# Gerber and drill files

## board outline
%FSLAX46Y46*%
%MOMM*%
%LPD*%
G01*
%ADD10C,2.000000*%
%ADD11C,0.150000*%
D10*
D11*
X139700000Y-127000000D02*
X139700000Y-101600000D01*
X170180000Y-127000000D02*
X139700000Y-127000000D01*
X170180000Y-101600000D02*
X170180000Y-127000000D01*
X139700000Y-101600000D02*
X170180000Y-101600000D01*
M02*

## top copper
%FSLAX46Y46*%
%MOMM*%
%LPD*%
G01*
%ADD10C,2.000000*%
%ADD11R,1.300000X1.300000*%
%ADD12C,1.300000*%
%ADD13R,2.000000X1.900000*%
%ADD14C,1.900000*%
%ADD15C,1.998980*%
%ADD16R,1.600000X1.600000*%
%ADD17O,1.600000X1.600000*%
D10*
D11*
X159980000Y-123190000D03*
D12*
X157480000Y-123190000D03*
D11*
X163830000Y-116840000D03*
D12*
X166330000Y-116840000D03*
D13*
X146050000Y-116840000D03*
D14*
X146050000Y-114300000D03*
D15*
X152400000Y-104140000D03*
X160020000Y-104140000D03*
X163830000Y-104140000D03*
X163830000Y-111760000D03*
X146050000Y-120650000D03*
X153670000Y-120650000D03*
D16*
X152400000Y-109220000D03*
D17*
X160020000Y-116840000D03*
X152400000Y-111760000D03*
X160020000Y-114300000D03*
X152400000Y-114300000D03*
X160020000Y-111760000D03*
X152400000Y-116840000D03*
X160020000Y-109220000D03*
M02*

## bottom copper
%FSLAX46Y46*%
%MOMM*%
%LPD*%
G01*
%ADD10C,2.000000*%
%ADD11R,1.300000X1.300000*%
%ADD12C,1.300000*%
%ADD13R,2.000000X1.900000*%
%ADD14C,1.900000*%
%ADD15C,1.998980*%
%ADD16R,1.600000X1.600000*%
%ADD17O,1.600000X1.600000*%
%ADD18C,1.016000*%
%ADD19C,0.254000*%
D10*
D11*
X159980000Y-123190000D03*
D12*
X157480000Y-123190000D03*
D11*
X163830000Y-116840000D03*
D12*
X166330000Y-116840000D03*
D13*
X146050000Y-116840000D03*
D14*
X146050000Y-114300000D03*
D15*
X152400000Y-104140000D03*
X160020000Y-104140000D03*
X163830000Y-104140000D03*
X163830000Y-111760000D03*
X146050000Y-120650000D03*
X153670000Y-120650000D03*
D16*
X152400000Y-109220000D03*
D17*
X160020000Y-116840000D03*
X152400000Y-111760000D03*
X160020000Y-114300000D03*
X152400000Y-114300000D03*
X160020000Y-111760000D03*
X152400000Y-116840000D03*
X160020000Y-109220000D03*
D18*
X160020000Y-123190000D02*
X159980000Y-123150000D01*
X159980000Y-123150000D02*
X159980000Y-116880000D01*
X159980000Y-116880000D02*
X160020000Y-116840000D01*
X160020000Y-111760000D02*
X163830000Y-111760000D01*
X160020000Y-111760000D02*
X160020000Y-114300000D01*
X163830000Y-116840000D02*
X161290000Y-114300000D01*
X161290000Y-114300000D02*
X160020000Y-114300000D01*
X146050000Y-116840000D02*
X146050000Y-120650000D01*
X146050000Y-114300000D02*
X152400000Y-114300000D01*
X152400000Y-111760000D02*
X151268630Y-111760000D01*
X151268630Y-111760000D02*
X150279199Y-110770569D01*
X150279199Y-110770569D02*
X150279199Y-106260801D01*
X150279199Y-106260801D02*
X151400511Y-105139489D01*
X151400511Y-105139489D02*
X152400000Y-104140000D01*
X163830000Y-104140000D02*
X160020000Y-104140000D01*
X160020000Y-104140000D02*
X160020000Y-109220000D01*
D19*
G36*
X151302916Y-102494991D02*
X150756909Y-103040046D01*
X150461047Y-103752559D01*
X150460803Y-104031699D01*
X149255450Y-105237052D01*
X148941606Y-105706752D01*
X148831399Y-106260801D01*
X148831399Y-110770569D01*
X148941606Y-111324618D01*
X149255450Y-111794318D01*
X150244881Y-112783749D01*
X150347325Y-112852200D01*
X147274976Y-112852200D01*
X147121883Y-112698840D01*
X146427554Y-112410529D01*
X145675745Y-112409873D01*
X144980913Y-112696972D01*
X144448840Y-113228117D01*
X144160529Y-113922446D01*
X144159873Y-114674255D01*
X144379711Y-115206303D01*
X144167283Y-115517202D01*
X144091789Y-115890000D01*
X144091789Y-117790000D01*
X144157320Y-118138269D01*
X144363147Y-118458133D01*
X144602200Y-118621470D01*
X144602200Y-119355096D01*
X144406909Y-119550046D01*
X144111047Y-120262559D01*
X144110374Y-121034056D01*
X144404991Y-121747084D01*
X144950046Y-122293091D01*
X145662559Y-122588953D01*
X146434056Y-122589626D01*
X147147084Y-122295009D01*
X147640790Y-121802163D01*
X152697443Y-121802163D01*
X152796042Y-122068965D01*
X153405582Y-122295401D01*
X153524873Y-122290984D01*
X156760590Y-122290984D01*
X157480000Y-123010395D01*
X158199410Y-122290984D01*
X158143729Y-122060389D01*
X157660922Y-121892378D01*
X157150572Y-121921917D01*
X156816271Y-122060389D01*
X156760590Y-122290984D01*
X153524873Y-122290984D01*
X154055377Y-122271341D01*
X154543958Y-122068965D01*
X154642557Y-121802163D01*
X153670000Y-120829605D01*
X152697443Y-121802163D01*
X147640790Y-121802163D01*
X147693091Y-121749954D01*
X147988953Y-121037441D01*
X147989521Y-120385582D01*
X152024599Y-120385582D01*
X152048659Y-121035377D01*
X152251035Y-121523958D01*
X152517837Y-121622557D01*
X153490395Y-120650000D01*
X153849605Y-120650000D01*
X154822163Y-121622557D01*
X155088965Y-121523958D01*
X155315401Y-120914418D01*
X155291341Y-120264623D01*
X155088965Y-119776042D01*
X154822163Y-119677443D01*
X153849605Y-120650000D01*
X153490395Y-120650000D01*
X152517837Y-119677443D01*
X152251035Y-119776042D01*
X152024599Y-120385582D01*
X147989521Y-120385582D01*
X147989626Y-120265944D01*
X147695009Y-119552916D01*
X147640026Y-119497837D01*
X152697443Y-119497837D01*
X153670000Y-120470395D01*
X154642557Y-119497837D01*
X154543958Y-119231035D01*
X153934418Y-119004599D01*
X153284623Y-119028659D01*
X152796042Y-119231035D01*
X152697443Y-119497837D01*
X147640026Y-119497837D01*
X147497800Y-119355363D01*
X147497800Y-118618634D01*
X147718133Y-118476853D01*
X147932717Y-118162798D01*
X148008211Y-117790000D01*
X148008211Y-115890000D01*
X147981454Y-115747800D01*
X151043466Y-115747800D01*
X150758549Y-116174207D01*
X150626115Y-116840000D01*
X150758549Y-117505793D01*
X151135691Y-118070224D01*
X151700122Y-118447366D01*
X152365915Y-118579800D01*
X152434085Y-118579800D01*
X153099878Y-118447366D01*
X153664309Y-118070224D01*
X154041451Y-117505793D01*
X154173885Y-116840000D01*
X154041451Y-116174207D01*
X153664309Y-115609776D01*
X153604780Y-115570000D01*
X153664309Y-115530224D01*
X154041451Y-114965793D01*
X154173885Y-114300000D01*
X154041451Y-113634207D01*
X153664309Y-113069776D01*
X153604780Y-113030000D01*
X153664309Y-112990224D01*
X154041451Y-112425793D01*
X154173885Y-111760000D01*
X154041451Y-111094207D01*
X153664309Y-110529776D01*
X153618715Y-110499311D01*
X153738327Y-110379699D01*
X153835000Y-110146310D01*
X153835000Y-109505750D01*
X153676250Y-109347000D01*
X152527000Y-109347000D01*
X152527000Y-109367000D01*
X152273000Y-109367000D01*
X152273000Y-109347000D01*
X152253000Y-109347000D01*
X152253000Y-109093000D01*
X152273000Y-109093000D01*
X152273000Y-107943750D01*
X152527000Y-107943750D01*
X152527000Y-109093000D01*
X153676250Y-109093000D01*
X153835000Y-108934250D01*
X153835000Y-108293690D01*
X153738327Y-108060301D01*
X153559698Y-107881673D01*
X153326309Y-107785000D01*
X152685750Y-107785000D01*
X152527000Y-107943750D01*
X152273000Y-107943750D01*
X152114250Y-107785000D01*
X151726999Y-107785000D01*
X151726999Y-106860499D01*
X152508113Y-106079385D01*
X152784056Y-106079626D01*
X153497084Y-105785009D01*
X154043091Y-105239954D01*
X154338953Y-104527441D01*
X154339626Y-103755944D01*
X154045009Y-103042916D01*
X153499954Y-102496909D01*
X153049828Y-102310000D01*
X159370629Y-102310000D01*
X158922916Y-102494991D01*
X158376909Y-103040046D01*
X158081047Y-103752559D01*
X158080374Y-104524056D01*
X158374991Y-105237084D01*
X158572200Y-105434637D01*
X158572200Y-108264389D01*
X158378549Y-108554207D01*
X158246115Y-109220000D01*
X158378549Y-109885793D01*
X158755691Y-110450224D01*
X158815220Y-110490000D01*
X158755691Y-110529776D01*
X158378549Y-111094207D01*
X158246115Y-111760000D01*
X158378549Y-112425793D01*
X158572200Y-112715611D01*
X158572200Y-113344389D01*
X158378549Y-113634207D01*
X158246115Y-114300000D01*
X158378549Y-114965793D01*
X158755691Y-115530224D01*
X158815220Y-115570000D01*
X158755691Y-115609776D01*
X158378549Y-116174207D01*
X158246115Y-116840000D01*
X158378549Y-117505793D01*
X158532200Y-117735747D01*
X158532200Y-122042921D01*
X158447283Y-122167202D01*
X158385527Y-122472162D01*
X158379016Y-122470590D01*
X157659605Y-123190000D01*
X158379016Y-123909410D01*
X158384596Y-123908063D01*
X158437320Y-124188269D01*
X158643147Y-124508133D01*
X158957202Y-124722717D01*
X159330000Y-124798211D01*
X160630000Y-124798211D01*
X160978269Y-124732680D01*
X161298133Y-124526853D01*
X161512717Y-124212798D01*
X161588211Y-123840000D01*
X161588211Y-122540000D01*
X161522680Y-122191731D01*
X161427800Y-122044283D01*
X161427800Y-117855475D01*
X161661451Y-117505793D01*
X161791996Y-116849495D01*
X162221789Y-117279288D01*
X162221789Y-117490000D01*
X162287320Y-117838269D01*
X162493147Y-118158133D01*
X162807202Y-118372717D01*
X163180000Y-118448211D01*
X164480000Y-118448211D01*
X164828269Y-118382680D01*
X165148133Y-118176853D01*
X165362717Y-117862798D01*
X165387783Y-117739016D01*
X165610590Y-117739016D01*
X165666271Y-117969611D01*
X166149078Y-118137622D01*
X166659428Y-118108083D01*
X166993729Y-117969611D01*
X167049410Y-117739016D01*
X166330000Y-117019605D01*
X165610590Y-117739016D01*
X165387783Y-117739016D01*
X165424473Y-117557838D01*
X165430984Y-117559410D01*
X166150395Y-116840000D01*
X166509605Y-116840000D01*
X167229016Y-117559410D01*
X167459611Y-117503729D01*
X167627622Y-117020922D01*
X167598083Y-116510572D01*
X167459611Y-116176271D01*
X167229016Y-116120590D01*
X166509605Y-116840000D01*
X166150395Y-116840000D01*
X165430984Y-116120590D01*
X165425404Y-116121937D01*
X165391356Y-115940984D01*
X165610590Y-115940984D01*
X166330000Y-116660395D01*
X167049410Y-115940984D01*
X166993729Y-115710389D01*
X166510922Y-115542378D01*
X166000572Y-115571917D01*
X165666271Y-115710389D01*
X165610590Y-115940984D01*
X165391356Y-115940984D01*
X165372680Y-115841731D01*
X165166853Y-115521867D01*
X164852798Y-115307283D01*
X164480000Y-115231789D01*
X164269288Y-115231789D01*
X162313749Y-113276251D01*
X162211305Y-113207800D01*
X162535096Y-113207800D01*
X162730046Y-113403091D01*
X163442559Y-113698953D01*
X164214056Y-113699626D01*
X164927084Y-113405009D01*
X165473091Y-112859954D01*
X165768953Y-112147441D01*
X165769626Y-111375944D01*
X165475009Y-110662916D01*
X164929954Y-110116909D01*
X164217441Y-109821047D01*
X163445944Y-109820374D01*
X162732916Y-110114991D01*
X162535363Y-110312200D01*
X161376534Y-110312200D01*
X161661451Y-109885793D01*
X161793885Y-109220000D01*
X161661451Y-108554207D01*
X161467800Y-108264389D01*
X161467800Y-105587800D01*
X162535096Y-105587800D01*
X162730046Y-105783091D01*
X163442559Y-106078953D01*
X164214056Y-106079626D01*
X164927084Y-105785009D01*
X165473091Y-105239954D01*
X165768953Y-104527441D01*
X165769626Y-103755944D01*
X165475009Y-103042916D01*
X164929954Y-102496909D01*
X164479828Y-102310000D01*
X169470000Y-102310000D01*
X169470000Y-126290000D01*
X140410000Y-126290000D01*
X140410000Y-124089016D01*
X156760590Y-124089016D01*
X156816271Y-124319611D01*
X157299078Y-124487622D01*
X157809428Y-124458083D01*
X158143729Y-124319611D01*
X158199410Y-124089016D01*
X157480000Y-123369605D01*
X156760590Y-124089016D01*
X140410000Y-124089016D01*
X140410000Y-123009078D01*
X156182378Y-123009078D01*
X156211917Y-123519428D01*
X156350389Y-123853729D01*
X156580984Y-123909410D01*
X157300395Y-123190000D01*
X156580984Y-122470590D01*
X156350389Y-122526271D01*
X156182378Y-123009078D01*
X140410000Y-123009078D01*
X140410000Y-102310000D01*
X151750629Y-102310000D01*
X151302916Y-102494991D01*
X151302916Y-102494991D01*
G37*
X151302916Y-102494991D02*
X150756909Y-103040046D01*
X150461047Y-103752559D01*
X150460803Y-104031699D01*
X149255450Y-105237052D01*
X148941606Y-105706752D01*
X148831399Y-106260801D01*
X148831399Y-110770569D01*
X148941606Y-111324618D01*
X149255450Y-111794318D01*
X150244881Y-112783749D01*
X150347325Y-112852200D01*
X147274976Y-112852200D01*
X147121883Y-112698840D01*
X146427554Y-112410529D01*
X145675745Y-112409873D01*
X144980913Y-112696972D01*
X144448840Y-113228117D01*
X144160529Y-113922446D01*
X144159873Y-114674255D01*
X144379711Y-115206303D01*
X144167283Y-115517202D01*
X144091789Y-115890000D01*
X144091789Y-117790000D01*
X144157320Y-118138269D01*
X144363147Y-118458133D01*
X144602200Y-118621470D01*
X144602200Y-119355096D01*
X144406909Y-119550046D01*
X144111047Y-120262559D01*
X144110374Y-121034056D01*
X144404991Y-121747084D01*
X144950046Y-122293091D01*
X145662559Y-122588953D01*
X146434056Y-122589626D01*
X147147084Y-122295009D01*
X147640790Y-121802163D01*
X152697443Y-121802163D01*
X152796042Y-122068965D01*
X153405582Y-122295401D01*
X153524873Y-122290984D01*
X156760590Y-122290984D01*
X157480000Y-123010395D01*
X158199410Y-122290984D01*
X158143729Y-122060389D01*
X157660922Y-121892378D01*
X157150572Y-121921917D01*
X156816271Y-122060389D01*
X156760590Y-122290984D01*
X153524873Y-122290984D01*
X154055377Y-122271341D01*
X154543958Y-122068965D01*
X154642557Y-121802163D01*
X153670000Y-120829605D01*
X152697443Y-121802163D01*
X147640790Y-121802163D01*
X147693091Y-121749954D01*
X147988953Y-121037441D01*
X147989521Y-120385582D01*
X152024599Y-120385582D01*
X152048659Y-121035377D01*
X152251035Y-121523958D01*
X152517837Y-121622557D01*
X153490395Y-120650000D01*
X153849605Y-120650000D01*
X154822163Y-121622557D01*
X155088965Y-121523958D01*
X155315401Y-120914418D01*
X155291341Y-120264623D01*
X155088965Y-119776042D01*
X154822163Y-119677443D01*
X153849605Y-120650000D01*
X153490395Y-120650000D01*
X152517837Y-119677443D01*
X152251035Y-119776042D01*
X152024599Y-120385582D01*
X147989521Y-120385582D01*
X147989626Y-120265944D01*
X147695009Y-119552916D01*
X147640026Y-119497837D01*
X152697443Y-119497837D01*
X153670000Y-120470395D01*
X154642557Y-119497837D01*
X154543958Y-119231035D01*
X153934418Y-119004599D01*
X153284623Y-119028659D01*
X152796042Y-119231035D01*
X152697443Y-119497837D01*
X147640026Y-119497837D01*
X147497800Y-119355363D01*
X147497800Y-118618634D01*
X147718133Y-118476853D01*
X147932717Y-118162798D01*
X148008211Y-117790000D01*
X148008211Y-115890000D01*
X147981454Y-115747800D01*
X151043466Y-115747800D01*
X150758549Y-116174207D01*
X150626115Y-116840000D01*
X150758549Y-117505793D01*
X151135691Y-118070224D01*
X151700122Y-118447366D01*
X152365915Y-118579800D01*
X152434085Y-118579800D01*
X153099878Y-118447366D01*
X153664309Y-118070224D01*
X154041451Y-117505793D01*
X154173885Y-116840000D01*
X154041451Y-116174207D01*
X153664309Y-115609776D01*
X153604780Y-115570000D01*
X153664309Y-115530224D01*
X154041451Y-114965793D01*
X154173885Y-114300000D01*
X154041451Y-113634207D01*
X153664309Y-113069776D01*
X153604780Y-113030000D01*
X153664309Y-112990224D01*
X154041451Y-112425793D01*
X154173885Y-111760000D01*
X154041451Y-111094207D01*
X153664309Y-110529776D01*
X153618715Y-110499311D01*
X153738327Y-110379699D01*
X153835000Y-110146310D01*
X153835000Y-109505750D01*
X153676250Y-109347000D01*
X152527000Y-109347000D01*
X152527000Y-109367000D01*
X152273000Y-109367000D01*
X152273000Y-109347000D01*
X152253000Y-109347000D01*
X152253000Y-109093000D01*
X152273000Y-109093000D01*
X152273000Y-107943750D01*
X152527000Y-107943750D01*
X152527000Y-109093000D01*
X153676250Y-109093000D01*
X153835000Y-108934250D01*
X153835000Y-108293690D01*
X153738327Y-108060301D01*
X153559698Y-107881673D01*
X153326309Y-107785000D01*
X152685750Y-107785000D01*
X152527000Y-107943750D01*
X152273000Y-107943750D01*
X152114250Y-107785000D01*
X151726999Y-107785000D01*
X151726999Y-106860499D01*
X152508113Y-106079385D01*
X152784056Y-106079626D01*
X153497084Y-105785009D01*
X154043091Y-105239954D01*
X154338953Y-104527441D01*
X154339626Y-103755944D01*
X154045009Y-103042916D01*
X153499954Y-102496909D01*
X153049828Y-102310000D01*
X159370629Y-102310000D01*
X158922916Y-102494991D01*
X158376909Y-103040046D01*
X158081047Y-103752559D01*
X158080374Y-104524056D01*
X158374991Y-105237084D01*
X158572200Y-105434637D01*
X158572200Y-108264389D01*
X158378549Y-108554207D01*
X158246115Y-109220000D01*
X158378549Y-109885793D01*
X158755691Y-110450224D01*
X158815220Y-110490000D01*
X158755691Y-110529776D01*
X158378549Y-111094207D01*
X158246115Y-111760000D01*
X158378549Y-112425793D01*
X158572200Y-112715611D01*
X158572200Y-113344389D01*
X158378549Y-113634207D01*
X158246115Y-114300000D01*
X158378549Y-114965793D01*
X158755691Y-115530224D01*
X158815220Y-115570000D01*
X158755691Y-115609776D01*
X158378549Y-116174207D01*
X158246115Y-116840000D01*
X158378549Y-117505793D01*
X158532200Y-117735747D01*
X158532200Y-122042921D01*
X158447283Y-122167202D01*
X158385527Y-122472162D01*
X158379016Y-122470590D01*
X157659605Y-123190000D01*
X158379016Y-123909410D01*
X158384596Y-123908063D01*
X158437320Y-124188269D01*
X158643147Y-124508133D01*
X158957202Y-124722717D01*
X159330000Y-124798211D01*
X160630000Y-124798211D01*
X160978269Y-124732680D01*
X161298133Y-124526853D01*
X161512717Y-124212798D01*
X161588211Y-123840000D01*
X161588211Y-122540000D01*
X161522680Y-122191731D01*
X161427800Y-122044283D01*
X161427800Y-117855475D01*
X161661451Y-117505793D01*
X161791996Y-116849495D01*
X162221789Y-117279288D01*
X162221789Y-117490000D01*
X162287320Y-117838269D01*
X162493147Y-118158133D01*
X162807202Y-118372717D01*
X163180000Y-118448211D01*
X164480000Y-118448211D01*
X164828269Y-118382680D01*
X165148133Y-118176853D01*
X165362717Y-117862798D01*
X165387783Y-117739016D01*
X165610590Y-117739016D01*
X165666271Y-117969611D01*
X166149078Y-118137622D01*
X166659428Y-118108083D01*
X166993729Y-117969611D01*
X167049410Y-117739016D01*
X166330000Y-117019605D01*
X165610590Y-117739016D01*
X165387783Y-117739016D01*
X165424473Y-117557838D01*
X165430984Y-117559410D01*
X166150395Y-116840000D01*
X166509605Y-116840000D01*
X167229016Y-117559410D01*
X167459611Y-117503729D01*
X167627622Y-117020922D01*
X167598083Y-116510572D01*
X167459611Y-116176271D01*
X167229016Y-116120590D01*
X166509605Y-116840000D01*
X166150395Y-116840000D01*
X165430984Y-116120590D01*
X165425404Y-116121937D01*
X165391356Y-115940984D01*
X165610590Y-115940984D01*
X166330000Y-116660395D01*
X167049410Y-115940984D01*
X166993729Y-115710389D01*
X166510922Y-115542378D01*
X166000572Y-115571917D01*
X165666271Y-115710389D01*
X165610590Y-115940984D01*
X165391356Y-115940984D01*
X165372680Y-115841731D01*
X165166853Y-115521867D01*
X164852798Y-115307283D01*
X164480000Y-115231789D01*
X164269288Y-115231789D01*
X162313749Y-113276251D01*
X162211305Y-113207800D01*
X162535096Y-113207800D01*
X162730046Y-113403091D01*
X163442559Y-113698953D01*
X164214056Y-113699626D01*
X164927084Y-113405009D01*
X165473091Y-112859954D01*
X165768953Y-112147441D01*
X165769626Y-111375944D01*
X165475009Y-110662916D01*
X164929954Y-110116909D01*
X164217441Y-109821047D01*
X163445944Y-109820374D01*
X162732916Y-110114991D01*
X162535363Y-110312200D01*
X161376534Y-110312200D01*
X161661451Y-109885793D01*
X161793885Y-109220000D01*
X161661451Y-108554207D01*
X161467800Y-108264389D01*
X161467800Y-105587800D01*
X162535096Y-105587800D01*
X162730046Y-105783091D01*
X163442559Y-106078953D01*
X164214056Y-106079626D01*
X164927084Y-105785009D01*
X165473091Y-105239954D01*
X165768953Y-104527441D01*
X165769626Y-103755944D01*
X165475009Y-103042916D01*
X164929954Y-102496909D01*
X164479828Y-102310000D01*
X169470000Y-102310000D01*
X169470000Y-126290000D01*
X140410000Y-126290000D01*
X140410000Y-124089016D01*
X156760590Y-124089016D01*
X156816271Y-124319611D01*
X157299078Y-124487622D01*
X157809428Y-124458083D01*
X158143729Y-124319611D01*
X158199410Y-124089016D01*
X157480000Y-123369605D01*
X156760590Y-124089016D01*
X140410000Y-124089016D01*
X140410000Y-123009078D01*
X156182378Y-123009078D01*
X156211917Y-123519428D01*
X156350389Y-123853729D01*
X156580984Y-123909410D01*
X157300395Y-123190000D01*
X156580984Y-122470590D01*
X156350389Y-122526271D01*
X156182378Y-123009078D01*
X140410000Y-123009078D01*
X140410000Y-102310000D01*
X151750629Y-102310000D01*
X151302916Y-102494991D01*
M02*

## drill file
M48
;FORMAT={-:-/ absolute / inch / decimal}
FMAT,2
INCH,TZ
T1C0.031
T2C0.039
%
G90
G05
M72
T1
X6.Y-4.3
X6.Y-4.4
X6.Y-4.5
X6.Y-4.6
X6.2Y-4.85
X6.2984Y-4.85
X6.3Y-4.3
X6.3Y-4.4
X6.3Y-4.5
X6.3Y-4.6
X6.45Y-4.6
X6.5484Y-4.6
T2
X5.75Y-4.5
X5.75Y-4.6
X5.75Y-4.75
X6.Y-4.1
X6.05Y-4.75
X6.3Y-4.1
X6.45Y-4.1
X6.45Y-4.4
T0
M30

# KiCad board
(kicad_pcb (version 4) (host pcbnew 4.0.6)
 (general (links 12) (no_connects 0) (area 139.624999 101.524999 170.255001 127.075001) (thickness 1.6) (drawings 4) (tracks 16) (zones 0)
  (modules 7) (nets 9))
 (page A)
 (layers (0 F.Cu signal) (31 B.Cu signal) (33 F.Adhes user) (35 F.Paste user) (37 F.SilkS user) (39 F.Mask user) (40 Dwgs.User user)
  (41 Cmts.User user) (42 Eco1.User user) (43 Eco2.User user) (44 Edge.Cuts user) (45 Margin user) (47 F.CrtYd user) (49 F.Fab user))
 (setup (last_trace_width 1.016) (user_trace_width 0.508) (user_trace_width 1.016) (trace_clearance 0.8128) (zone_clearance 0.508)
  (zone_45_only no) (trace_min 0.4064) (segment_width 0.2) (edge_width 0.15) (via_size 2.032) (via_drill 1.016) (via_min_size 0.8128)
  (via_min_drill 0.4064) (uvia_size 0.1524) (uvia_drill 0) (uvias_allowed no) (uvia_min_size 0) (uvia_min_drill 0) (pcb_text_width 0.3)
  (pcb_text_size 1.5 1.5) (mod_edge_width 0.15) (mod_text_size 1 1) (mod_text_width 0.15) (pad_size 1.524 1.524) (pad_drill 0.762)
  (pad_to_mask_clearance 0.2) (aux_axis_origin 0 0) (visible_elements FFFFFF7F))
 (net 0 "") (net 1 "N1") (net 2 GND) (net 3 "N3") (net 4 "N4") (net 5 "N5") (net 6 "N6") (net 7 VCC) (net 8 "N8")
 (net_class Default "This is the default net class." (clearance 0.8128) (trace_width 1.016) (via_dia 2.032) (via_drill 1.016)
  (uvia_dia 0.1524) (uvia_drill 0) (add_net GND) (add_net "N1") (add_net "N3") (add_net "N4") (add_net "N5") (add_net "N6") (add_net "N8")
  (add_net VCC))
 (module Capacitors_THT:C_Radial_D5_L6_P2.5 (layer F.Cu) (at 159.98 123.19 180)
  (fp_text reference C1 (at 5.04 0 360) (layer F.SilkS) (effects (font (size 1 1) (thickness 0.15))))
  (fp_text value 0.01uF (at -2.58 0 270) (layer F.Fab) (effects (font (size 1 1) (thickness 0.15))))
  (pad 1 thru_hole rect (at 0 0 180) (size 1.3 1.3) (drill 0.8) (layers *.Cu *.Mask) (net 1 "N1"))
  (pad 2 thru_hole circle (at 2.5 0 180) (size 1.3 1.3) (drill 0.8) (layers *.Cu *.Mask) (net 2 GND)))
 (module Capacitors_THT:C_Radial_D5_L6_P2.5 (layer F.Cu) (at 163.83 116.84)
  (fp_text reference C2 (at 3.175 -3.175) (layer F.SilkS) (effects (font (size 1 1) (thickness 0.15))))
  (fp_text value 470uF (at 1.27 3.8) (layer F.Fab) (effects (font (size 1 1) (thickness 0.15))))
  (pad 1 thru_hole rect (at 0 0) (size 1.3 1.3) (drill 0.8) (layers *.Cu *.Mask) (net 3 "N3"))
  (pad 2 thru_hole circle (at 2.5 0) (size 1.3 1.3) (drill 0.8) (layers *.Cu *.Mask) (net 2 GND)))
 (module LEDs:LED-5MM (layer F.Cu) (at 146.05 116.84 90)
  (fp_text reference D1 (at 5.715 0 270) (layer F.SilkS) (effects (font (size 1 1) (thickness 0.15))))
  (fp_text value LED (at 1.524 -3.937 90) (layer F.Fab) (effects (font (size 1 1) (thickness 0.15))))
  (pad 1 thru_hole rect (at 0 0 180) (size 2 1.9) (drill 1.00076) (layers *.Cu *.Mask) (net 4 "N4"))
  (pad 2 thru_hole circle (at 2.54 0 90) (size 1.9 1.9) (drill 1.00076) (layers *.Cu *.Mask) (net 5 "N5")))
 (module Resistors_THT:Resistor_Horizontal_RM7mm (layer F.Cu) (at 152.4 104.14)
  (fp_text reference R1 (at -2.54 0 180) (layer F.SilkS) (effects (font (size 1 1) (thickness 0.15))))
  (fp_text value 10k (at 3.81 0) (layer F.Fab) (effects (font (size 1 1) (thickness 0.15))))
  (pad 1 thru_hole circle (at 0 0) (size 1.99898 1.99898) (drill 1.00076) (layers *.Cu *.SilkS *.Mask) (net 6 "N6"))
  (pad 2 thru_hole circle (at 7.62 0) (size 1.99898 1.99898) (drill 1.00076) (layers *.Cu *.SilkS *.Mask) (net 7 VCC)))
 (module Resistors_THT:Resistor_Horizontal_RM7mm (layer F.Cu) (at 163.83 104.14 270)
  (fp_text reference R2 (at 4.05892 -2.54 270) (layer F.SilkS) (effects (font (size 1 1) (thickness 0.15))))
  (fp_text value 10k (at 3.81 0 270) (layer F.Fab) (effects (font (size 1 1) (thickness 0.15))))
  (pad 1 thru_hole circle (at 0 0 270) (size 1.99898 1.99898) (drill 1.00076) (layers *.Cu *.SilkS *.Mask) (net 7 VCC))
  (pad 2 thru_hole circle (at 7.62 0 270) (size 1.99898 1.99898) (drill 1.00076) (layers *.Cu *.SilkS *.Mask) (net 3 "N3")))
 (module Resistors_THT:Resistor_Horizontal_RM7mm (layer F.Cu) (at 146.05 120.65)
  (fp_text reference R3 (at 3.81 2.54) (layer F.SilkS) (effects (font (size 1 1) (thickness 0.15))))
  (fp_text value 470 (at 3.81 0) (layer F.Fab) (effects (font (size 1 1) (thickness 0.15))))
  (pad 1 thru_hole circle (at 0 0) (size 1.99898 1.99898) (drill 1.00076) (layers *.Cu *.SilkS *.Mask) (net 4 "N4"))
  (pad 2 thru_hole circle (at 7.62 0) (size 1.99898 1.99898) (drill 1.00076) (layers *.Cu *.SilkS *.Mask) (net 2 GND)))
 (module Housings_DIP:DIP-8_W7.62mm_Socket (layer F.Cu) (at 152.4 109.22)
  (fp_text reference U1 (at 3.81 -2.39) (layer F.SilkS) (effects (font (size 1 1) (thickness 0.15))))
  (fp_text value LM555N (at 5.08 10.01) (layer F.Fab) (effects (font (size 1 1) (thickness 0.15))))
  (pad 1 thru_hole rect (at 0 0) (size 1.6 1.6) (drill 0.8) (layers *.Cu *.Mask) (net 2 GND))
  (pad 5 thru_hole oval (at 7.62 7.62) (size 1.6 1.6) (drill 0.8) (layers *.Cu *.Mask) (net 1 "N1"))
  (pad 2 thru_hole oval (at 0 2.54) (size 1.6 1.6) (drill 0.8) (layers *.Cu *.Mask) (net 6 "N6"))
  (pad 6 thru_hole oval (at 7.62 5.08) (size 1.6 1.6) (drill 0.8) (layers *.Cu *.Mask) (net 3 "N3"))
  (pad 3 thru_hole oval (at 0 5.08) (size 1.6 1.6) (drill 0.8) (layers *.Cu *.Mask) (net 5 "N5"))
  (pad 7 thru_hole oval (at 7.62 2.54) (size 1.6 1.6) (drill 0.8) (layers *.Cu *.Mask) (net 3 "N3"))
  (pad 4 thru_hole oval (at 0 7.62) (size 1.6 1.6) (drill 0.8) (layers *.Cu *.Mask) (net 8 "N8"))
  (pad 8 thru_hole oval (at 7.62 0) (size 1.6 1.6) (drill 0.8) (layers *.Cu *.Mask) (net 7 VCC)))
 (gr_line (start 139.7 127) (end 139.7 101.6) (layer Edge.Cuts) (width 0.15))
 (gr_line (start 170.18 127) (end 139.7 127) (layer Edge.Cuts) (width 0.15))
 (gr_line (start 170.18 101.6) (end 170.18 127) (layer Edge.Cuts) (width 0.15))
 (gr_line (start 139.7 101.6) (end 170.18 101.6) (layer Edge.Cuts) (width 0.15))
 (segment (start 160.02 123.19) (end 159.98 123.15) (width 1.016) (layer B.Cu) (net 1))
 (segment (start 159.98 123.15) (end 159.98 116.88) (width 1.016) (layer B.Cu) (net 1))
 (segment (start 159.98 116.88) (end 160.02 116.84) (width 1.016) (layer B.Cu) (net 1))
 (segment (start 160.02 111.76) (end 163.83 111.76) (width 1.016) (layer B.Cu) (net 3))
 (segment (start 160.02 111.76) (end 160.02 114.3) (width 1.016) (layer B.Cu) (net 3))
 (segment (start 163.83 116.84) (end 161.29 114.3) (width 1.016) (layer B.Cu) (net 3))
 (segment (start 161.29 114.3) (end 160.02 114.3) (width 1.016) (layer B.Cu) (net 3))
 (segment (start 146.05 116.84) (end 146.05 120.65) (width 1.016) (layer B.Cu) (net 4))
 (segment (start 146.05 114.3) (end 152.4 114.3) (width 1.016) (layer B.Cu) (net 5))
 (segment (start 152.4 111.76) (end 151.26863 111.76) (width 1.016) (layer B.Cu) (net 6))
 (segment (start 151.26863 111.76) (end 150.279199 110.770569) (width 1.016) (layer B.Cu) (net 6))
 (segment (start 150.279199 110.770569) (end 150.279199 106.260801) (width 1.016) (layer B.Cu) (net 6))
 (segment (start 150.279199 106.260801) (end 151.400511 105.139489) (width 1.016) (layer B.Cu) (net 6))
 (segment (start 151.400511 105.139489) (end 152.4 104.14) (width 1.016) (layer B.Cu) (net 6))
 (segment (start 163.83 104.14) (end 160.02 104.14) (width 1.016) (layer B.Cu) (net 7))
 (segment (start 160.02 104.14) (end 160.02 109.22) (width 1.016) (layer B.Cu) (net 7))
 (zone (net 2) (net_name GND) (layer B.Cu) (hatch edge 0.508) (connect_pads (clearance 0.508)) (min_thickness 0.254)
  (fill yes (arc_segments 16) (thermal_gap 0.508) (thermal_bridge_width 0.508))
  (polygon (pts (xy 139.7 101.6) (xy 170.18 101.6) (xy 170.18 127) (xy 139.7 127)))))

